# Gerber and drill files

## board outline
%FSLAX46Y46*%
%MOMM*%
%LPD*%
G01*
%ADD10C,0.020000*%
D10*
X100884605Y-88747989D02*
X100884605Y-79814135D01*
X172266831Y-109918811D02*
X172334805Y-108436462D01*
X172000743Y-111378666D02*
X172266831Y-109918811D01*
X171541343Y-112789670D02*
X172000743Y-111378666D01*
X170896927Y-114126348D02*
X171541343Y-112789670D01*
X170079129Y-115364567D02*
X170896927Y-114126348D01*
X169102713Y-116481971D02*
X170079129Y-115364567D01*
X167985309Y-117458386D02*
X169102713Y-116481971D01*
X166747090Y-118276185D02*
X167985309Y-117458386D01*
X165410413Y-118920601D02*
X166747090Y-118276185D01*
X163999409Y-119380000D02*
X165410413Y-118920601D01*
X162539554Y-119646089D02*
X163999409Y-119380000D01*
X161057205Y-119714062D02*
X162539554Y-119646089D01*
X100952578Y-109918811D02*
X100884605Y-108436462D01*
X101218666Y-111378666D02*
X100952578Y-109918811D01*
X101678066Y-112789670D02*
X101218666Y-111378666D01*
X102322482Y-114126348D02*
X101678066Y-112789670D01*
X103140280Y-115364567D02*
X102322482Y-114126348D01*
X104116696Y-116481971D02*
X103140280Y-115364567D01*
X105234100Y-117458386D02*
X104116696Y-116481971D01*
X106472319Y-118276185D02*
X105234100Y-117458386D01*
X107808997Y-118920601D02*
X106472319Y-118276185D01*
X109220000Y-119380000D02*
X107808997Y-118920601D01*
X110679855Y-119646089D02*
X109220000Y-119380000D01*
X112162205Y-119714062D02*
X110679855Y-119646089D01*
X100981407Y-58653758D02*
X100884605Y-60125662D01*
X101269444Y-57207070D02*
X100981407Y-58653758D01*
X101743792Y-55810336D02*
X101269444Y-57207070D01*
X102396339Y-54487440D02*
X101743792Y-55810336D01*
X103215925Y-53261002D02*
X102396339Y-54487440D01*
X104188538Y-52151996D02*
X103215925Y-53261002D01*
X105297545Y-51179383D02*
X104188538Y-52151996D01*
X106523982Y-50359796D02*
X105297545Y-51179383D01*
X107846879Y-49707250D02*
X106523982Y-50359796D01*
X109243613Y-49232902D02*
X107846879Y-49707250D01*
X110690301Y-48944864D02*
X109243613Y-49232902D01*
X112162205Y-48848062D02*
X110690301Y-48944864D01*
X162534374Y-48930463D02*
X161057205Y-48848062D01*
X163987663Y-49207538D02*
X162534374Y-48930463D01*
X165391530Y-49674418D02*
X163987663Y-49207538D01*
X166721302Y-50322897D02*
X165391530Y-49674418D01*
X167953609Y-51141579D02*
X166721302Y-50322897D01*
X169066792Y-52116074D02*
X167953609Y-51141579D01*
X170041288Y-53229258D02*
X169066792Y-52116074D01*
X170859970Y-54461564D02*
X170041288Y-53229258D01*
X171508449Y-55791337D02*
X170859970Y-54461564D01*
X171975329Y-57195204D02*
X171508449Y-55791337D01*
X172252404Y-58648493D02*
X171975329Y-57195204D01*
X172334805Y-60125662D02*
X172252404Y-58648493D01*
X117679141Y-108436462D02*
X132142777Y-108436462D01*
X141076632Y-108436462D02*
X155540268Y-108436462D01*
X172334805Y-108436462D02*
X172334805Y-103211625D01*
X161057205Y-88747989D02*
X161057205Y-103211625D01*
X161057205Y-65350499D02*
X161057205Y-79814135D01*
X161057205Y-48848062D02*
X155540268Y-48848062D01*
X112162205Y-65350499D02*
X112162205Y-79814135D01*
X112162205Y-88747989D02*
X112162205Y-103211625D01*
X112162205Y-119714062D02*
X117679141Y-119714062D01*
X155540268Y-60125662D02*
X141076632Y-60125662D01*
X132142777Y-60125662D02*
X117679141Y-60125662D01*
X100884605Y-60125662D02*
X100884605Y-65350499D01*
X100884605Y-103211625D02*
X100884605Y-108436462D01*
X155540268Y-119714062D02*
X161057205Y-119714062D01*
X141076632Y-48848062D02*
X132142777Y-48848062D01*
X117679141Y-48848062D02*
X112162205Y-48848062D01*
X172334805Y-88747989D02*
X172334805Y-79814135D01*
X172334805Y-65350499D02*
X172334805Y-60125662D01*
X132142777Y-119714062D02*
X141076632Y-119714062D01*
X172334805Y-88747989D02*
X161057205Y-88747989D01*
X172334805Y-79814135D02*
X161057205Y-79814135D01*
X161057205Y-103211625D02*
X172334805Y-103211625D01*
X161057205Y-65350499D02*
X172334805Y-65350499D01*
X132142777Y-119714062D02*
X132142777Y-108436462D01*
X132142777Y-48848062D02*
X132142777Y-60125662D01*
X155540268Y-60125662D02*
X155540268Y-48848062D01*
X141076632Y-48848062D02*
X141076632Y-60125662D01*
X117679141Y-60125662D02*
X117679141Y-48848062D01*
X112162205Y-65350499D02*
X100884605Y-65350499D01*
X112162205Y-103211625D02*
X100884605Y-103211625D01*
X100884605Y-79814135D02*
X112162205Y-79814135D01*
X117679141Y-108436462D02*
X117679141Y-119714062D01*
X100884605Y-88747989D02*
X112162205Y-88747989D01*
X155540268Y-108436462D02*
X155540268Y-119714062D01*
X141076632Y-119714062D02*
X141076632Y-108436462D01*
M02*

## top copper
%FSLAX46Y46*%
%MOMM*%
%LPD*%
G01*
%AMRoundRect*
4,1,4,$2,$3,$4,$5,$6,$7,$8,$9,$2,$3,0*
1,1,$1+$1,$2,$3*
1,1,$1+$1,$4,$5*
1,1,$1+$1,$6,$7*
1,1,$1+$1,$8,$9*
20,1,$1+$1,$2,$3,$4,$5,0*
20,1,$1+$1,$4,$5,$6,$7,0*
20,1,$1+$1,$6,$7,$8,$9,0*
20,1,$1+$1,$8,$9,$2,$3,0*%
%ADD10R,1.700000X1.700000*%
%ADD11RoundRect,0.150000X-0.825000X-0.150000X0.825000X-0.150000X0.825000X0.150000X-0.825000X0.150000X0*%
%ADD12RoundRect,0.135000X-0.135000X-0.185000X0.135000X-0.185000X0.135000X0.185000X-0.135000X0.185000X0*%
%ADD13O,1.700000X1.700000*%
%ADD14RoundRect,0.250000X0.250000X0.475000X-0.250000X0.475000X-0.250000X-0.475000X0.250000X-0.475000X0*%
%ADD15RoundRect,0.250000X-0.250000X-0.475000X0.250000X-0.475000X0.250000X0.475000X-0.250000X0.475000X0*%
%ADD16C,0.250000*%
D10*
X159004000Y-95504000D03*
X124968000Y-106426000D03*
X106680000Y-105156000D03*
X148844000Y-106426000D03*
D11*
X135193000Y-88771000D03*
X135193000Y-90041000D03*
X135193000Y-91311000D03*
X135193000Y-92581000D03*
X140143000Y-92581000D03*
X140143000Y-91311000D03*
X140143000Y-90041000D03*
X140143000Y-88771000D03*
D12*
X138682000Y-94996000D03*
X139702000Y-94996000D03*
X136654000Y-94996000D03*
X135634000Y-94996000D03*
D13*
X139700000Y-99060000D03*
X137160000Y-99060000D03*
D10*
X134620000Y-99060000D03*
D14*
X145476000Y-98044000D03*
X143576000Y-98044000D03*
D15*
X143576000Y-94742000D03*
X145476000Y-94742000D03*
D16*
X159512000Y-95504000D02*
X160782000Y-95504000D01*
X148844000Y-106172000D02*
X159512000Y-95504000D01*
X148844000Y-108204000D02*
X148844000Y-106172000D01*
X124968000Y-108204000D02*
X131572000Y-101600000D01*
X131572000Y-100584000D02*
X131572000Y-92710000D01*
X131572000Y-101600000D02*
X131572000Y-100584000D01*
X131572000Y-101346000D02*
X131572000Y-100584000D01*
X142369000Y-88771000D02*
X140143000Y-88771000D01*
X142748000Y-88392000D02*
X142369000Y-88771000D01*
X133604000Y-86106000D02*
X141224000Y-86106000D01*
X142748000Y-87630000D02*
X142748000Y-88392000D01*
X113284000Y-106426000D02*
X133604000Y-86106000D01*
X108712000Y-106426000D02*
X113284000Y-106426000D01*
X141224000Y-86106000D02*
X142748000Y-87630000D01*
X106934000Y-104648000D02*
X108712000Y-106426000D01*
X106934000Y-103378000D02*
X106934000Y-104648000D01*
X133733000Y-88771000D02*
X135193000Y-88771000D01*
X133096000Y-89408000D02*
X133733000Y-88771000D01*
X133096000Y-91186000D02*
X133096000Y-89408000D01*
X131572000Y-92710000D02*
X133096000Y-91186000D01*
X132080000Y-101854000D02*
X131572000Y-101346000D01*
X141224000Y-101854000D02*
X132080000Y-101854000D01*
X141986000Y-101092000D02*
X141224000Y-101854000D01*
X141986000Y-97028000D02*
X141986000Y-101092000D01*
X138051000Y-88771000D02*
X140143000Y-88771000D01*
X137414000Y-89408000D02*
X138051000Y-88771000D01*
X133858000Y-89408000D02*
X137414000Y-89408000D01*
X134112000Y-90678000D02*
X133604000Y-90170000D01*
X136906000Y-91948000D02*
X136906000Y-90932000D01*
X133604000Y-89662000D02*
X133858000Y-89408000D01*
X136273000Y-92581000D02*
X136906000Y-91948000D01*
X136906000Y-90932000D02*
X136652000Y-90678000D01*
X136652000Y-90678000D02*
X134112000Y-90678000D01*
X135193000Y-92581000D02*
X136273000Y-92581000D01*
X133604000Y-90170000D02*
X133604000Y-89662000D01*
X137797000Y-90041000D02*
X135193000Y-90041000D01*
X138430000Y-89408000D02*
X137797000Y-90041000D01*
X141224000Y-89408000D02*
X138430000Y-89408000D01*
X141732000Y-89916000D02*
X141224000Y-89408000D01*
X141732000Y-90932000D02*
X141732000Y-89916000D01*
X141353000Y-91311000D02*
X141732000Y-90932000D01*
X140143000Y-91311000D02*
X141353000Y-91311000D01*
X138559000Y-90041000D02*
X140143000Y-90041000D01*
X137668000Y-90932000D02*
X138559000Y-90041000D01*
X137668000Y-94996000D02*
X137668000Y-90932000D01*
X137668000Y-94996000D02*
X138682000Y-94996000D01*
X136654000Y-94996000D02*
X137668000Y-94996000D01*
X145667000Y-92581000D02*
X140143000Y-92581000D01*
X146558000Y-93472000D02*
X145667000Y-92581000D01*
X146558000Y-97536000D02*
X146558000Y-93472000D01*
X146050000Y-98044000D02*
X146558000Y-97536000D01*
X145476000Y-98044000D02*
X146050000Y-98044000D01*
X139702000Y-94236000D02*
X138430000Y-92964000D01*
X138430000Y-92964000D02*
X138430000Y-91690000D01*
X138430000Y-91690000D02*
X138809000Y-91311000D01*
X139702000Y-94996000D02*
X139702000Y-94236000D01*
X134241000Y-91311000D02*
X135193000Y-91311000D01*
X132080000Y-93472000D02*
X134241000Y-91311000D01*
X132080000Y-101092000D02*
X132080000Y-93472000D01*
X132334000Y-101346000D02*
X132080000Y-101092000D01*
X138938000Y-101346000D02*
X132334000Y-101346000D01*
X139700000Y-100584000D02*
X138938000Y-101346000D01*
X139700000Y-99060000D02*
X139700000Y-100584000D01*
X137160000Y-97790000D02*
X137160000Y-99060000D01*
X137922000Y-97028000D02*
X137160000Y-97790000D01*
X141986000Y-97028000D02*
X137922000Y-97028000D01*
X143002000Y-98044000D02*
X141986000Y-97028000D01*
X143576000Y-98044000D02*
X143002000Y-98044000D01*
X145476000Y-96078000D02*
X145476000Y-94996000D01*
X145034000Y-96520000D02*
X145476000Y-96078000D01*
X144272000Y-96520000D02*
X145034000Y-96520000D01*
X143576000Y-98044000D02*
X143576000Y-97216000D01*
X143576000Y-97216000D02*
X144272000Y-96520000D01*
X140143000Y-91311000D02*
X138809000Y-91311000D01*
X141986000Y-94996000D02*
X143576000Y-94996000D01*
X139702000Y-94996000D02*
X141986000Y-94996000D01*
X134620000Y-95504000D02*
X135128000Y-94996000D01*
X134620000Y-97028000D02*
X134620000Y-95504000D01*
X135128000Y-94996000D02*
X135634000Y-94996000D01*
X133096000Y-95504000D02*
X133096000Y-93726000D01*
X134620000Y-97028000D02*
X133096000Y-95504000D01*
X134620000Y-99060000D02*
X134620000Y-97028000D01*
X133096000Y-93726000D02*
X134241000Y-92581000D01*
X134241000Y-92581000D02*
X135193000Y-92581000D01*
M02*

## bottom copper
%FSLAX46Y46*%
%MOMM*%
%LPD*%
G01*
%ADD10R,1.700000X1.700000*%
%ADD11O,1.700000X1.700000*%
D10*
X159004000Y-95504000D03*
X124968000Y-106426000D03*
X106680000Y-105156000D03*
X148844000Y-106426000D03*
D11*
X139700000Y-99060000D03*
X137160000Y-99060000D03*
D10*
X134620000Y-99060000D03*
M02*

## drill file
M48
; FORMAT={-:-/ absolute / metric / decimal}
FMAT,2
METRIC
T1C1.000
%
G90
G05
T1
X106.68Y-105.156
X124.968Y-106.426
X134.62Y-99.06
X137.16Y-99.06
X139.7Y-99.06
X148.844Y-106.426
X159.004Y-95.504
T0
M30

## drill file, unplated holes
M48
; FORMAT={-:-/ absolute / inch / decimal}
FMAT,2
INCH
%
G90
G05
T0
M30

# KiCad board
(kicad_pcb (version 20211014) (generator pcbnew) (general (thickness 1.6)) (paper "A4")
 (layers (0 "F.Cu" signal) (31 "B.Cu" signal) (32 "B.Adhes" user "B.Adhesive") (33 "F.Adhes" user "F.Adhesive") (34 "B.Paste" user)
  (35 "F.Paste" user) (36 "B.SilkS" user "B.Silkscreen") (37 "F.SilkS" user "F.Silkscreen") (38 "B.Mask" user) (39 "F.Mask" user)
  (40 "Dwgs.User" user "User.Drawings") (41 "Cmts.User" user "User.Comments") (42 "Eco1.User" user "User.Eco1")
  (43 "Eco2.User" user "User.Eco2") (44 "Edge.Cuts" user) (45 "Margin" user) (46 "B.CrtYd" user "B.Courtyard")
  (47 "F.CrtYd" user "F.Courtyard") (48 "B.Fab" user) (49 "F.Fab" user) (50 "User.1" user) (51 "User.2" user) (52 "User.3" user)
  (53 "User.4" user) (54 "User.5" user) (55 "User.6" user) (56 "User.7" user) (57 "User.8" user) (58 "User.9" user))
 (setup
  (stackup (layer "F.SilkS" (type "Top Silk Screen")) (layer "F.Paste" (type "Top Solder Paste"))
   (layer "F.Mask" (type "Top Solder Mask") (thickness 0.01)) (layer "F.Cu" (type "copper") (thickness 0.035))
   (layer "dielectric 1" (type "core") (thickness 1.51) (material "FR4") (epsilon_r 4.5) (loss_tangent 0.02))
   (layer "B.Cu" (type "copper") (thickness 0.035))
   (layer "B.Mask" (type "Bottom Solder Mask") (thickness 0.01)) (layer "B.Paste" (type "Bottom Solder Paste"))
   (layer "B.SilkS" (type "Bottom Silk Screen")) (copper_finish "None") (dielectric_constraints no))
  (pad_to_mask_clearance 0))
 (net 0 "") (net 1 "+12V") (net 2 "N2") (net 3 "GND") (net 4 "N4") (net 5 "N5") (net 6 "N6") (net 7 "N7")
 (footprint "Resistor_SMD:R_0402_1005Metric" (layer "F.Cu") (at 136.144 94.996)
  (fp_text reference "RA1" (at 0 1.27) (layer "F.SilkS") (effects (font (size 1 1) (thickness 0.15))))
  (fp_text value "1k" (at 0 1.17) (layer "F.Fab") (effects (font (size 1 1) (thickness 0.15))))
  (pad "1" smd roundrect (at -0.51 0) (size 0.54 0.64) (layers "F.Cu" "F.Paste" "F.Mask") (roundrect_rratio 0.25) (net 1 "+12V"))
  (pad "2" smd roundrect (at 0.51 0) (size 0.54 0.64) (layers "F.Cu" "F.Paste" "F.Mask") (roundrect_rratio 0.25) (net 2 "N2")))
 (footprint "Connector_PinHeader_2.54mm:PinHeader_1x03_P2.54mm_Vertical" (layer "F.Cu") (at 134.62 99.06 90)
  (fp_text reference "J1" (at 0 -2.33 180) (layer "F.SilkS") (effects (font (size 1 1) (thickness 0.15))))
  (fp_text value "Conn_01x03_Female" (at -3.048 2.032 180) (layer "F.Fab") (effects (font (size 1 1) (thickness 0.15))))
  (pad "1" thru_hole rect (at 0 0 90) (size 1.7 1.7) (drill 1) (layers *.Cu *.Mask) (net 1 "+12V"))
  (pad "2" thru_hole oval (at 0 2.54 90) (size 1.7 1.7) (drill 1) (layers *.Cu *.Mask) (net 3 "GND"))
  (pad "3" thru_hole oval (at 0 5.08 90) (size 1.7 1.7) (drill 1) (layers *.Cu *.Mask) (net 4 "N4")))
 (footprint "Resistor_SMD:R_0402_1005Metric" (layer "F.Cu") (at 139.192 94.996)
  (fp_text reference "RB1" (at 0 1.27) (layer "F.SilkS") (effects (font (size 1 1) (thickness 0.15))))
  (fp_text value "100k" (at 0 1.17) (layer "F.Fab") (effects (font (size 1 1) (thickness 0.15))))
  (pad "1" smd roundrect (at -0.51 0) (size 0.54 0.64) (layers "F.Cu" "F.Paste" "F.Mask") (roundrect_rratio 0.25) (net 2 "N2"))
  (pad "2" smd roundrect (at 0.51 0) (size 0.54 0.64) (layers "F.Cu" "F.Paste" "F.Mask") (roundrect_rratio 0.25) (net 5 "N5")))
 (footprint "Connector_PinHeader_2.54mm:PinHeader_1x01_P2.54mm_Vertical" (layer "F.Cu") (at 106.68 105.156 180)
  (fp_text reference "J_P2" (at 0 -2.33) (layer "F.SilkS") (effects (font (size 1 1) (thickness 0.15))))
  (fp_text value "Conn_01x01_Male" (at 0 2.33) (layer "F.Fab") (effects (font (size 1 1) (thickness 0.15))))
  (pad "1" thru_hole rect (at 0 0 180) (size 1.7 1.7) (drill 1) (layers *.Cu *.Mask) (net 1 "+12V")))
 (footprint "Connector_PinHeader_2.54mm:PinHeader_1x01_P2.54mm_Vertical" (layer "F.Cu") (at 148.844 106.426)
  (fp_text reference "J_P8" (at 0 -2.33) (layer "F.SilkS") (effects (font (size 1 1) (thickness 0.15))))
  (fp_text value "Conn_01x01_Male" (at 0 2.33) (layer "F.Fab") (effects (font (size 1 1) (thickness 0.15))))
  (pad "1" thru_hole rect (at 0 0) (size 1.7 1.7) (drill 1) (layers *.Cu *.Mask) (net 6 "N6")))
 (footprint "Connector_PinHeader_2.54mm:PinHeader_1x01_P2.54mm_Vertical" (layer "F.Cu") (at 124.968 106.426)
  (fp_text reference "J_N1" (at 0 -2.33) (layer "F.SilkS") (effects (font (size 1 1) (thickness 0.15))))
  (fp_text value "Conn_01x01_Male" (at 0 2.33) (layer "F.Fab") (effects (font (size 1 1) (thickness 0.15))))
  (pad "1" thru_hole rect (at 0 0) (size 1.7 1.7) (drill 1) (layers *.Cu *.Mask) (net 3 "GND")))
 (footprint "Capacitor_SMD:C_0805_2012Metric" (layer "F.Cu") (at 144.526 98.044 180)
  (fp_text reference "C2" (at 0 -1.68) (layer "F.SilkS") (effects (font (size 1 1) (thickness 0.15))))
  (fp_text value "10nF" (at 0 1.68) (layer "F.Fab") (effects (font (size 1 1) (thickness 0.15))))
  (pad "1" smd roundrect (at -0.95 0 180) (size 1 1.45) (layers "F.Cu" "F.Paste" "F.Mask") (roundrect_rratio 0.25) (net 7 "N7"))
  (pad "2" smd roundrect (at 0.95 0 180) (size 1 1.45) (layers "F.Cu" "F.Paste" "F.Mask") (roundrect_rratio 0.25) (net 3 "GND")))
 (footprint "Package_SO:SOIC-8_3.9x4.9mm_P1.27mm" (layer "F.Cu") (at 137.668 90.676)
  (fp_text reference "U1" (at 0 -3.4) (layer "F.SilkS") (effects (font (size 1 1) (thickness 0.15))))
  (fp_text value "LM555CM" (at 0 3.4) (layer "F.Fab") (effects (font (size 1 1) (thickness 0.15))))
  (pad "1" smd roundrect (at -2.475 -1.905) (size 1.95 0.6) (layers "F.Cu" "F.Paste" "F.Mask") (roundrect_rratio 0.25) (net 3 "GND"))
  (pad "2" smd roundrect (at -2.475 -0.635) (size 1.95 0.6) (layers "F.Cu" "F.Paste" "F.Mask") (roundrect_rratio 0.25) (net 5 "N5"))
  (pad "3" smd roundrect (at -2.475 0.635) (size 1.95 0.6) (layers "F.Cu" "F.Paste" "F.Mask") (roundrect_rratio 0.25) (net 4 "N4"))
  (pad "4" smd roundrect (at -2.475 1.905) (size 1.95 0.6) (layers "F.Cu" "F.Paste" "F.Mask") (roundrect_rratio 0.25) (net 1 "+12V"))
  (pad "5" smd roundrect (at 2.475 1.905) (size 1.95 0.6) (layers "F.Cu" "F.Paste" "F.Mask") (roundrect_rratio 0.25) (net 7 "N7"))
  (pad "6" smd roundrect (at 2.475 0.635) (size 1.95 0.6) (layers "F.Cu" "F.Paste" "F.Mask") (roundrect_rratio 0.25) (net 5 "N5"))
  (pad "7" smd roundrect (at 2.475 -0.635) (size 1.95 0.6) (layers "F.Cu" "F.Paste" "F.Mask") (roundrect_rratio 0.25) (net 2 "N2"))
  (pad "8" smd roundrect (at 2.475 -1.905) (size 1.95 0.6) (layers "F.Cu" "F.Paste" "F.Mask") (roundrect_rratio 0.25) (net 1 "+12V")))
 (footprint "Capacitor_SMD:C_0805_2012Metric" (layer "F.Cu") (at 144.526 94.742)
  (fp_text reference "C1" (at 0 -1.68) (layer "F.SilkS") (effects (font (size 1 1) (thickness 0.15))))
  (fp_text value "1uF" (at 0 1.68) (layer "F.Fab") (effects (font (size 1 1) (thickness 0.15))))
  (pad "1" smd roundrect (at -0.95 0) (size 1 1.45) (layers "F.Cu" "F.Paste" "F.Mask") (roundrect_rratio 0.25) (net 5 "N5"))
  (pad "2" smd roundrect (at 0.95 0) (size 1 1.45) (layers "F.Cu" "F.Paste" "F.Mask") (roundrect_rratio 0.25) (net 3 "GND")))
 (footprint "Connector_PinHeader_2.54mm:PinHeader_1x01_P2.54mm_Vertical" (layer "F.Cu") (at 159.004 95.504 90)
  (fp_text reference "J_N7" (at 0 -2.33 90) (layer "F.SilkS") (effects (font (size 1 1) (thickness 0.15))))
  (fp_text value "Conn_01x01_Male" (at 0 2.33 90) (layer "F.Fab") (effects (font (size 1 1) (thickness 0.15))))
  (pad "1" thru_hole rect (at 0 0 90) (size 1.7 1.7) (drill 1) (layers *.Cu *.Mask) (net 6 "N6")))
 (gr_line (start 170.85997 54.461564) (end 170.041288 53.229258) (layer "Edge.Cuts") (width 0.02))
 (gr_line (start 141.076632 108.436462) (end 155.540268 108.436462) (layer "Edge.Cuts") (width 0.02))
 (gr_line (start 105.2341 117.458386) (end 104.116696 116.481971) (layer "Edge.Cuts") (width 0.02))
 (gr_line (start 170.896927 114.126348) (end 171.541343 112.78967) (layer "Edge.Cuts") (width 0.02))
 (gr_line (start 166.721302 50.322897) (end 165.39153 49.674418) (layer "Edge.Cuts") (width 0.02))
 (gr_line (start 107.846879 49.70725) (end 106.523982 50.359796) (layer "Edge.Cuts") (width 0.02))
 (gr_line (start 170.041288 53.229258) (end 169.066792 52.116074) (layer "Edge.Cuts") (width 0.02))
 (gr_line (start 172.334805 79.814135) (end 161.057205 79.814135) (layer "Edge.Cuts") (width 0.02))
 (gr_line (start 117.679141 60.125662) (end 117.679141 48.848062) (layer "Edge.Cuts") (width 0.02))
 (gr_line (start 172.334805 65.350499) (end 172.334805 60.125662) (layer "Edge.Cuts") (width 0.02))
 (gr_line (start 171.508449 55.791337) (end 170.85997 54.461564) (layer "Edge.Cuts") (width 0.02))
 (gr_line (start 161.057205 65.350499) (end 161.057205 79.814135) (layer "Edge.Cuts") (width 0.02))
 (gr_line (start 172.334805 88.747989) (end 161.057205 88.747989) (layer "Edge.Cuts") (width 0.02))
 (gr_line (start 172.334805 88.747989) (end 172.334805 79.814135) (layer "Edge.Cuts") (width 0.02))
 (gr_line (start 155.540268 119.714062) (end 161.057205 119.714062) (layer "Edge.Cuts") (width 0.02))
 (gr_line (start 110.690301 48.944864) (end 109.243613 49.232902) (layer "Edge.Cuts") (width 0.02))
 (gr_line (start 172.252404 58.648493) (end 171.975329 57.195204) (layer "Edge.Cuts") (width 0.02))
 (gr_line (start 104.116696 116.481971) (end 103.14028 115.364567) (layer "Edge.Cuts") (width 0.02))
 (gr_line (start 172.000743 111.378666) (end 172.266831 109.918811) (layer "Edge.Cuts") (width 0.02))
 (gr_line (start 170.079129 115.364567) (end 170.896927 114.126348) (layer "Edge.Cuts") (width 0.02))
 (gr_line (start 100.884605 103.211625) (end 100.884605 108.436462) (layer "Edge.Cuts") (width 0.02))
 (gr_line (start 105.297545 51.179383) (end 104.188538 52.151996) (layer "Edge.Cuts") (width 0.02))
 (gr_line (start 102.322482 114.126348) (end 101.678066 112.78967) (layer "Edge.Cuts") (width 0.02))
 (gr_line (start 112.162205 88.747989) (end 112.162205 103.211625) (layer "Edge.Cuts") (width 0.02))
 (gr_line (start 167.953609 51.141579) (end 166.721302 50.322897) (layer "Edge.Cuts") (width 0.02))
 (gr_line (start 112.162205 48.848062) (end 110.690301 48.944864) (layer "Edge.Cuts") (width 0.02))
 (gr_line (start 117.679141 108.436462) (end 132.142777 108.436462) (layer "Edge.Cuts") (width 0.02))
 (gr_line (start 132.142777 48.848062) (end 132.142777 60.125662) (layer "Edge.Cuts") (width 0.02))
 (gr_line (start 102.396339 54.48744) (end 101.743792 55.810336) (layer "Edge.Cuts") (width 0.02))
 (gr_line (start 132.142777 119.714062) (end 141.076632 119.714062) (layer "Edge.Cuts") (width 0.02))
 (gr_line (start 117.679141 48.848062) (end 112.162205 48.848062) (layer "Edge.Cuts") (width 0.02))
 (gr_line (start 112.162205 65.350499) (end 100.884605 65.350499) (layer "Edge.Cuts") (width 0.02))
 (gr_line (start 112.162205 119.714062) (end 110.679855 119.646089) (layer "Edge.Cuts") (width 0.02))
 (gr_line (start 132.142777 60.125662) (end 117.679141 60.125662) (layer "Edge.Cuts") (width 0.02))
 (gr_line (start 161.057205 119.714062) (end 162.539554 119.646089) (layer "Edge.Cuts") (width 0.02))
 (gr_line (start 141.076632 48.848062) (end 141.076632 60.125662) (layer "Edge.Cuts") (width 0.02))
 (gr_line (start 172.334805 60.125662) (end 172.252404 58.648493) (layer "Edge.Cuts") (width 0.02))
 (gr_line (start 141.076632 119.714062) (end 141.076632 108.436462) (layer "Edge.Cuts") (width 0.02))
 (gr_line (start 169.102713 116.481971) (end 170.079129 115.364567) (layer "Edge.Cuts") (width 0.02))
 (gr_line (start 141.076632 48.848062) (end 132.142777 48.848062) (layer "Edge.Cuts") (width 0.02))
 (gr_line (start 162.539554 119.646089) (end 163.999409 119.38) (layer "Edge.Cuts") (width 0.02))
 (gr_line (start 106.472319 118.276185) (end 105.2341 117.458386) (layer "Edge.Cuts") (width 0.02))
 (gr_line (start 163.987663 49.207538) (end 162.534374 48.930463) (layer "Edge.Cuts") (width 0.02))
 (gr_line (start 172.266831 109.918811) (end 172.334805 108.436462) (layer "Edge.Cuts") (width 0.02))
 (gr_line (start 161.057205 88.747989) (end 161.057205 103.211625) (layer "Edge.Cuts") (width 0.02))
 (gr_line (start 155.540268 60.125662) (end 141.076632 60.125662) (layer "Edge.Cuts") (width 0.02))
 (gr_line (start 101.218666 111.378666) (end 100.952578 109.918811) (layer "Edge.Cuts") (width 0.02))
 (gr_line (start 100.884605 88.747989) (end 100.884605 79.814135) (layer "Edge.Cuts") (width 0.02))
 (gr_line (start 112.162205 119.714062) (end 117.679141 119.714062) (layer "Edge.Cuts") (width 0.02))
 (gr_line (start 117.679141 108.436462) (end 117.679141 119.714062) (layer "Edge.Cuts") (width 0.02))
 (gr_line (start 104.188538 52.151996) (end 103.215925 53.261002) (layer "Edge.Cuts") (width 0.02))
 (gr_line (start 162.534374 48.930463) (end 161.057205 48.848062) (layer "Edge.Cuts") (width 0.02))
 (gr_line (start 100.981407 58.653758) (end 100.884605 60.125662) (layer "Edge.Cuts") (width 0.02))
 (gr_line (start 172.334805 108.436462) (end 172.334805 103.211625) (layer "Edge.Cuts") (width 0.02))
 (gr_line (start 100.952578 109.918811) (end 100.884605 108.436462) (layer "Edge.Cuts") (width 0.02))
 (gr_line (start 106.523982 50.359796) (end 105.297545 51.179383) (layer "Edge.Cuts") (width 0.02))
 (gr_line (start 169.066792 52.116074) (end 167.953609 51.141579) (layer "Edge.Cuts") (width 0.02))
 (gr_line (start 109.22 119.38) (end 107.808997 118.920601) (layer "Edge.Cuts") (width 0.02))
 (gr_line (start 167.985309 117.458386) (end 169.102713 116.481971) (layer "Edge.Cuts") (width 0.02))
 (gr_line (start 101.743792 55.810336) (end 101.269444 57.20707) (layer "Edge.Cuts") (width 0.02))
 (gr_line (start 166.74709 118.276185) (end 167.985309 117.458386) (layer "Edge.Cuts") (width 0.02))
 (gr_line (start 161.057205 65.350499) (end 172.334805 65.350499) (layer "Edge.Cuts") (width 0.02))
 (gr_line (start 132.142777 119.714062) (end 132.142777 108.436462) (layer "Edge.Cuts") (width 0.02))
 (gr_line (start 155.540268 60.125662) (end 155.540268 48.848062) (layer "Edge.Cuts") (width 0.02))
 (gr_line (start 161.057205 48.848062) (end 155.540268 48.848062) (layer "Edge.Cuts") (width 0.02))
 (gr_line (start 171.541343 112.78967) (end 172.000743 111.378666) (layer "Edge.Cuts") (width 0.02))
 (gr_line (start 100.884605 88.747989) (end 112.162205 88.747989) (layer "Edge.Cuts") (width 0.02))
 (gr_line (start 103.14028 115.364567) (end 102.322482 114.126348) (layer "Edge.Cuts") (width 0.02))
 (gr_line (start 101.269444 57.20707) (end 100.981407 58.653758) (layer "Edge.Cuts") (width 0.02))
 (gr_line (start 161.057205 103.211625) (end 172.334805 103.211625) (layer "Edge.Cuts") (width 0.02))
 (gr_line (start 109.243613 49.232902) (end 107.846879 49.70725) (layer "Edge.Cuts") (width 0.02))
 (gr_line (start 163.999409 119.38) (end 165.410413 118.920601) (layer "Edge.Cuts") (width 0.02))
 (gr_line (start 103.215925 53.261002) (end 102.396339 54.48744) (layer "Edge.Cuts") (width 0.02))
 (gr_line (start 155.540268 108.436462) (end 155.540268 119.714062) (layer "Edge.Cuts") (width 0.02))
 (gr_line (start 110.679855 119.646089) (end 109.22 119.38) (layer "Edge.Cuts") (width 0.02))
 (gr_line (start 100.884605 60.125662) (end 100.884605 65.350499) (layer "Edge.Cuts") (width 0.02))
 (gr_line (start 101.678066 112.78967) (end 101.218666 111.378666) (layer "Edge.Cuts") (width 0.02))
 (gr_line (start 165.39153 49.674418) (end 163.987663 49.207538) (layer "Edge.Cuts") (width 0.02))
 (gr_line (start 107.808997 118.920601) (end 106.472319 118.276185) (layer "Edge.Cuts") (width 0.02))
 (gr_line (start 112.162205 103.211625) (end 100.884605 103.211625) (layer "Edge.Cuts") (width 0.02))
 (gr_line (start 112.162205 65.350499) (end 112.162205 79.814135) (layer "Edge.Cuts") (width 0.02))
 (gr_line (start 100.884605 79.814135) (end 112.162205 79.814135) (layer "Edge.Cuts") (width 0.02))
 (gr_line (start 165.410413 118.920601) (end 166.74709 118.276185) (layer "Edge.Cuts") (width 0.02))
 (gr_line (start 171.975329 57.195204) (end 171.508449 55.791337) (layer "Edge.Cuts") (width 0.02))
 (segment (start 140.143 91.311) (end 138.809 91.311) (width 0.25) (layer "F.Cu") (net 5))
 (segment (start 138.43 91.69) (end 138.809 91.311) (width 0.25) (layer "F.Cu") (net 5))
 (segment (start 139.702 94.996) (end 139.702 94.236) (width 0.25) (layer "F.Cu") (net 5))
 (segment (start 138.43 92.964) (end 138.43 91.69) (width 0.25) (layer "F.Cu") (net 5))
 (segment (start 141.224 89.408) (end 138.43 89.408) (width 0.25) (layer "F.Cu") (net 5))
 (segment (start 139.702 94.996) (end 141.986 94.996) (width 0.25) (layer "F.Cu") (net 5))
 (segment (start 139.702 94.236) (end 138.43 92.964) (width 0.25) (layer "F.Cu") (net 5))
 (segment (start 141.732 90.932) (end 141.732 89.916) (width 0.25) (layer "F.Cu") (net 5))
 (segment (start 138.43 89.408) (end 137.797 90.041) (width 0.25) (layer "F.Cu") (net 5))
 (segment (start 137.797 90.041) (end 135.193 90.041) (width 0.25) (layer "F.Cu") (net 5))
 (segment (start 141.986 94.996) (end 143.576 94.996) (width 0.25) (layer "F.Cu") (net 5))
 (segment (start 141.732 89.916) (end 141.224 89.408) (width 0.25) (layer "F.Cu") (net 5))
 (segment (start 141.353 91.311) (end 141.732 90.932) (width 0.25) (layer "F.Cu") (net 5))
 (segment (start 140.143 91.311) (end 141.353 91.311) (width 0.25) (layer "F.Cu") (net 5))
 (segment (start 131.572 100.584) (end 131.572 92.71) (width 0.25) (layer "F.Cu") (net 3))
 (segment (start 131.572 101.346) (end 131.572 100.584) (width 0.25) (layer "F.Cu") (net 3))
 (segment (start 132.08 101.854) (end 131.572 101.346) (width 0.25) (layer "F.Cu") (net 3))
 (segment (start 143.576 97.216) (end 144.272 96.52) (width 0.25) (layer "F.Cu") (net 3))
 (segment (start 141.986 97.028) (end 141.986 101.092) (width 0.25) (layer "F.Cu") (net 3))
 (segment (start 141.986 101.092) (end 141.224 101.854) (width 0.25) (layer "F.Cu") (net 3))
 (segment (start 133.733 88.771) (end 135.193 88.771) (width 0.25) (layer "F.Cu") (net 3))
 (segment (start 131.572 101.6) (end 131.572 100.584) (width 0.25) (layer "F.Cu") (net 3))
 (segment (start 143.576 98.044) (end 143.576 97.216) (width 0.25) (layer "F.Cu") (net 3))
 (segment (start 145.034 96.52) (end 145.476 96.078) (width 0.25) (layer "F.Cu") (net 3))
 (segment (start 137.16 97.79) (end 137.16 99.06) (width 0.25) (layer "F.Cu") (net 3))
 (segment (start 133.096 91.186) (end 133.096 89.408) (width 0.25) (layer "F.Cu") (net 3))
 (segment (start 145.476 96.078) (end 145.476 94.996) (width 0.25) (layer "F.Cu") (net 3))
 (segment (start 141.224 101.854) (end 132.08 101.854) (width 0.25) (layer "F.Cu") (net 3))
 (segment (start 124.968 108.204) (end 131.572 101.6) (width 0.25) (layer "F.Cu") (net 3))
 (segment (start 137.922 97.028) (end 137.16 97.79) (width 0.25) (layer "F.Cu") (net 3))
 (segment (start 141.986 97.028) (end 137.922 97.028) (width 0.25) (layer "F.Cu") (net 3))
 (segment (start 131.572 92.71) (end 133.096 91.186) (width 0.25) (layer "F.Cu") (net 3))
 (segment (start 133.096 89.408) (end 133.733 88.771) (width 0.25) (layer "F.Cu") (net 3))
 (segment (start 144.272 96.52) (end 145.034 96.52) (width 0.25) (layer "F.Cu") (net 3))
 (segment (start 143.002 98.044) (end 141.986 97.028) (width 0.25) (layer "F.Cu") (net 3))
 (segment (start 143.576 98.044) (end 143.002 98.044) (width 0.25) (layer "F.Cu") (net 3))
 (segment (start 145.476 98.044) (end 146.05 98.044) (width 0.25) (layer "F.Cu") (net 7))
 (segment (start 146.558 97.536) (end 146.558 93.472) (width 0.25) (layer "F.Cu") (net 7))
 (segment (start 146.05 98.044) (end 146.558 97.536) (width 0.25) (layer "F.Cu") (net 7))
 (segment (start 145.667 92.581) (end 140.143 92.581) (width 0.25) (layer "F.Cu") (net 7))
 (segment (start 146.558 93.472) (end 145.667 92.581) (width 0.25) (layer "F.Cu") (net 7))
 (segment (start 133.604 89.662) (end 133.858 89.408) (width 0.25) (layer "F.Cu") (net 1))
 (segment (start 142.748 88.392) (end 142.369 88.771) (width 0.25) (layer "F.Cu") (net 1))
 (segment (start 142.369 88.771) (end 140.143 88.771) (width 0.25) (layer "F.Cu") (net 1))
 (segment (start 134.62 97.028) (end 133.096 95.504) (width 0.25) (layer "F.Cu") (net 1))
 (segment (start 136.652 90.678) (end 134.112 90.678) (width 0.25) (layer "F.Cu") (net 1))
 (segment (start 135.128 94.996) (end 135.634 94.996) (width 0.25) (layer "F.Cu") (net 1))
 (segment (start 106.934 103.378) (end 106.934 104.648) (width 0.25) (layer "F.Cu") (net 1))
 (segment (start 133.604 90.17) (end 133.604 89.662) (width 0.25) (layer "F.Cu") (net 1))
 (segment (start 137.414 89.408) (end 138.051 88.771) (width 0.25) (layer "F.Cu") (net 1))
 (segment (start 133.096 93.726) (end 134.241 92.581) (width 0.25) (layer "F.Cu") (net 1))
 (segment (start 134.112 90.678) (end 133.604 90.17) (width 0.25) (layer "F.Cu") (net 1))
 (segment (start 138.051 88.771) (end 140.143 88.771) (width 0.25) (layer "F.Cu") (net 1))
 (segment (start 135.193 92.581) (end 136.273 92.581) (width 0.25) (layer "F.Cu") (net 1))
 (segment (start 134.241 92.581) (end 135.193 92.581) (width 0.25) (layer "F.Cu") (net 1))
 (segment (start 134.62 95.504) (end 135.128 94.996) (width 0.25) (layer "F.Cu") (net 1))
 (segment (start 133.096 95.504) (end 133.096 93.726) (width 0.25) (layer "F.Cu") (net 1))
 (segment (start 141.224 86.106) (end 142.748 87.63) (width 0.25) (layer "F.Cu") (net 1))
 (segment (start 134.62 99.06) (end 134.62 97.028) (width 0.25) (layer "F.Cu") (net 1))
 (segment (start 133.604 86.106) (end 141.224 86.106) (width 0.25) (layer "F.Cu") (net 1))
 (segment (start 113.284 106.426) (end 133.604 86.106) (width 0.25) (layer "F.Cu") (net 1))
 (segment (start 142.748 87.63) (end 142.748 88.392) (width 0.25) (layer "F.Cu") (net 1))
 (segment (start 136.906 90.932) (end 136.652 90.678) (width 0.25) (layer "F.Cu") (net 1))
 (segment (start 134.62 97.028) (end 134.62 95.504) (width 0.25) (layer "F.Cu") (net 1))
 (segment (start 136.273 92.581) (end 136.906 91.948) (width 0.25) (layer "F.Cu") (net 1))
 (segment (start 136.906 91.948) (end 136.906 90.932) (width 0.25) (layer "F.Cu") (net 1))
 (segment (start 106.934 104.648) (end 108.712 106.426) (width 0.25) (layer "F.Cu") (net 1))
 (segment (start 133.858 89.408) (end 137.414 89.408) (width 0.25) (layer "F.Cu") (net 1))
 (segment (start 108.712 106.426) (end 113.284 106.426) (width 0.25) (layer "F.Cu") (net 1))
 (segment (start 138.938 101.346) (end 132.334 101.346) (width 0.25) (layer "F.Cu") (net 4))
 (segment (start 132.08 101.092) (end 132.08 93.472) (width 0.25) (layer "F.Cu") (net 4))
 (segment (start 132.334 101.346) (end 132.08 101.092) (width 0.25) (layer "F.Cu") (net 4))
 (segment (start 134.241 91.311) (end 135.193 91.311) (width 0.25) (layer "F.Cu") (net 4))
 (segment (start 132.08 93.472) (end 134.241 91.311) (width 0.25) (layer "F.Cu") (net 4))
 (segment (start 139.7 99.06) (end 139.7 100.584) (width 0.25) (layer "F.Cu") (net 4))
 (segment (start 139.7 100.584) (end 138.938 101.346) (width 0.25) (layer "F.Cu") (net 4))
 (segment (start 138.559 90.041) (end 140.143 90.041) (width 0.25) (layer "F.Cu") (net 2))
 (segment (start 137.668 94.996) (end 138.682 94.996) (width 0.25) (layer "F.Cu") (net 2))
 (segment (start 136.654 94.996) (end 137.668 94.996) (width 0.25) (layer "F.Cu") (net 2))
 (segment (start 137.668 90.932) (end 138.559 90.041) (width 0.25) (layer "F.Cu") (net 2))
 (segment (start 137.668 94.996) (end 137.668 90.932) (width 0.25) (layer "F.Cu") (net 2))
 (segment (start 148.844 108.204) (end 148.844 106.172) (width 0.25) (layer "F.Cu") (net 6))
 (segment (start 148.844 106.172) (end 159.512 95.504) (width 0.25) (layer "F.Cu") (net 6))
 (segment (start 159.512 95.504) (end 160.782 95.504) (width 0.25) (layer "F.Cu") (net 6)))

